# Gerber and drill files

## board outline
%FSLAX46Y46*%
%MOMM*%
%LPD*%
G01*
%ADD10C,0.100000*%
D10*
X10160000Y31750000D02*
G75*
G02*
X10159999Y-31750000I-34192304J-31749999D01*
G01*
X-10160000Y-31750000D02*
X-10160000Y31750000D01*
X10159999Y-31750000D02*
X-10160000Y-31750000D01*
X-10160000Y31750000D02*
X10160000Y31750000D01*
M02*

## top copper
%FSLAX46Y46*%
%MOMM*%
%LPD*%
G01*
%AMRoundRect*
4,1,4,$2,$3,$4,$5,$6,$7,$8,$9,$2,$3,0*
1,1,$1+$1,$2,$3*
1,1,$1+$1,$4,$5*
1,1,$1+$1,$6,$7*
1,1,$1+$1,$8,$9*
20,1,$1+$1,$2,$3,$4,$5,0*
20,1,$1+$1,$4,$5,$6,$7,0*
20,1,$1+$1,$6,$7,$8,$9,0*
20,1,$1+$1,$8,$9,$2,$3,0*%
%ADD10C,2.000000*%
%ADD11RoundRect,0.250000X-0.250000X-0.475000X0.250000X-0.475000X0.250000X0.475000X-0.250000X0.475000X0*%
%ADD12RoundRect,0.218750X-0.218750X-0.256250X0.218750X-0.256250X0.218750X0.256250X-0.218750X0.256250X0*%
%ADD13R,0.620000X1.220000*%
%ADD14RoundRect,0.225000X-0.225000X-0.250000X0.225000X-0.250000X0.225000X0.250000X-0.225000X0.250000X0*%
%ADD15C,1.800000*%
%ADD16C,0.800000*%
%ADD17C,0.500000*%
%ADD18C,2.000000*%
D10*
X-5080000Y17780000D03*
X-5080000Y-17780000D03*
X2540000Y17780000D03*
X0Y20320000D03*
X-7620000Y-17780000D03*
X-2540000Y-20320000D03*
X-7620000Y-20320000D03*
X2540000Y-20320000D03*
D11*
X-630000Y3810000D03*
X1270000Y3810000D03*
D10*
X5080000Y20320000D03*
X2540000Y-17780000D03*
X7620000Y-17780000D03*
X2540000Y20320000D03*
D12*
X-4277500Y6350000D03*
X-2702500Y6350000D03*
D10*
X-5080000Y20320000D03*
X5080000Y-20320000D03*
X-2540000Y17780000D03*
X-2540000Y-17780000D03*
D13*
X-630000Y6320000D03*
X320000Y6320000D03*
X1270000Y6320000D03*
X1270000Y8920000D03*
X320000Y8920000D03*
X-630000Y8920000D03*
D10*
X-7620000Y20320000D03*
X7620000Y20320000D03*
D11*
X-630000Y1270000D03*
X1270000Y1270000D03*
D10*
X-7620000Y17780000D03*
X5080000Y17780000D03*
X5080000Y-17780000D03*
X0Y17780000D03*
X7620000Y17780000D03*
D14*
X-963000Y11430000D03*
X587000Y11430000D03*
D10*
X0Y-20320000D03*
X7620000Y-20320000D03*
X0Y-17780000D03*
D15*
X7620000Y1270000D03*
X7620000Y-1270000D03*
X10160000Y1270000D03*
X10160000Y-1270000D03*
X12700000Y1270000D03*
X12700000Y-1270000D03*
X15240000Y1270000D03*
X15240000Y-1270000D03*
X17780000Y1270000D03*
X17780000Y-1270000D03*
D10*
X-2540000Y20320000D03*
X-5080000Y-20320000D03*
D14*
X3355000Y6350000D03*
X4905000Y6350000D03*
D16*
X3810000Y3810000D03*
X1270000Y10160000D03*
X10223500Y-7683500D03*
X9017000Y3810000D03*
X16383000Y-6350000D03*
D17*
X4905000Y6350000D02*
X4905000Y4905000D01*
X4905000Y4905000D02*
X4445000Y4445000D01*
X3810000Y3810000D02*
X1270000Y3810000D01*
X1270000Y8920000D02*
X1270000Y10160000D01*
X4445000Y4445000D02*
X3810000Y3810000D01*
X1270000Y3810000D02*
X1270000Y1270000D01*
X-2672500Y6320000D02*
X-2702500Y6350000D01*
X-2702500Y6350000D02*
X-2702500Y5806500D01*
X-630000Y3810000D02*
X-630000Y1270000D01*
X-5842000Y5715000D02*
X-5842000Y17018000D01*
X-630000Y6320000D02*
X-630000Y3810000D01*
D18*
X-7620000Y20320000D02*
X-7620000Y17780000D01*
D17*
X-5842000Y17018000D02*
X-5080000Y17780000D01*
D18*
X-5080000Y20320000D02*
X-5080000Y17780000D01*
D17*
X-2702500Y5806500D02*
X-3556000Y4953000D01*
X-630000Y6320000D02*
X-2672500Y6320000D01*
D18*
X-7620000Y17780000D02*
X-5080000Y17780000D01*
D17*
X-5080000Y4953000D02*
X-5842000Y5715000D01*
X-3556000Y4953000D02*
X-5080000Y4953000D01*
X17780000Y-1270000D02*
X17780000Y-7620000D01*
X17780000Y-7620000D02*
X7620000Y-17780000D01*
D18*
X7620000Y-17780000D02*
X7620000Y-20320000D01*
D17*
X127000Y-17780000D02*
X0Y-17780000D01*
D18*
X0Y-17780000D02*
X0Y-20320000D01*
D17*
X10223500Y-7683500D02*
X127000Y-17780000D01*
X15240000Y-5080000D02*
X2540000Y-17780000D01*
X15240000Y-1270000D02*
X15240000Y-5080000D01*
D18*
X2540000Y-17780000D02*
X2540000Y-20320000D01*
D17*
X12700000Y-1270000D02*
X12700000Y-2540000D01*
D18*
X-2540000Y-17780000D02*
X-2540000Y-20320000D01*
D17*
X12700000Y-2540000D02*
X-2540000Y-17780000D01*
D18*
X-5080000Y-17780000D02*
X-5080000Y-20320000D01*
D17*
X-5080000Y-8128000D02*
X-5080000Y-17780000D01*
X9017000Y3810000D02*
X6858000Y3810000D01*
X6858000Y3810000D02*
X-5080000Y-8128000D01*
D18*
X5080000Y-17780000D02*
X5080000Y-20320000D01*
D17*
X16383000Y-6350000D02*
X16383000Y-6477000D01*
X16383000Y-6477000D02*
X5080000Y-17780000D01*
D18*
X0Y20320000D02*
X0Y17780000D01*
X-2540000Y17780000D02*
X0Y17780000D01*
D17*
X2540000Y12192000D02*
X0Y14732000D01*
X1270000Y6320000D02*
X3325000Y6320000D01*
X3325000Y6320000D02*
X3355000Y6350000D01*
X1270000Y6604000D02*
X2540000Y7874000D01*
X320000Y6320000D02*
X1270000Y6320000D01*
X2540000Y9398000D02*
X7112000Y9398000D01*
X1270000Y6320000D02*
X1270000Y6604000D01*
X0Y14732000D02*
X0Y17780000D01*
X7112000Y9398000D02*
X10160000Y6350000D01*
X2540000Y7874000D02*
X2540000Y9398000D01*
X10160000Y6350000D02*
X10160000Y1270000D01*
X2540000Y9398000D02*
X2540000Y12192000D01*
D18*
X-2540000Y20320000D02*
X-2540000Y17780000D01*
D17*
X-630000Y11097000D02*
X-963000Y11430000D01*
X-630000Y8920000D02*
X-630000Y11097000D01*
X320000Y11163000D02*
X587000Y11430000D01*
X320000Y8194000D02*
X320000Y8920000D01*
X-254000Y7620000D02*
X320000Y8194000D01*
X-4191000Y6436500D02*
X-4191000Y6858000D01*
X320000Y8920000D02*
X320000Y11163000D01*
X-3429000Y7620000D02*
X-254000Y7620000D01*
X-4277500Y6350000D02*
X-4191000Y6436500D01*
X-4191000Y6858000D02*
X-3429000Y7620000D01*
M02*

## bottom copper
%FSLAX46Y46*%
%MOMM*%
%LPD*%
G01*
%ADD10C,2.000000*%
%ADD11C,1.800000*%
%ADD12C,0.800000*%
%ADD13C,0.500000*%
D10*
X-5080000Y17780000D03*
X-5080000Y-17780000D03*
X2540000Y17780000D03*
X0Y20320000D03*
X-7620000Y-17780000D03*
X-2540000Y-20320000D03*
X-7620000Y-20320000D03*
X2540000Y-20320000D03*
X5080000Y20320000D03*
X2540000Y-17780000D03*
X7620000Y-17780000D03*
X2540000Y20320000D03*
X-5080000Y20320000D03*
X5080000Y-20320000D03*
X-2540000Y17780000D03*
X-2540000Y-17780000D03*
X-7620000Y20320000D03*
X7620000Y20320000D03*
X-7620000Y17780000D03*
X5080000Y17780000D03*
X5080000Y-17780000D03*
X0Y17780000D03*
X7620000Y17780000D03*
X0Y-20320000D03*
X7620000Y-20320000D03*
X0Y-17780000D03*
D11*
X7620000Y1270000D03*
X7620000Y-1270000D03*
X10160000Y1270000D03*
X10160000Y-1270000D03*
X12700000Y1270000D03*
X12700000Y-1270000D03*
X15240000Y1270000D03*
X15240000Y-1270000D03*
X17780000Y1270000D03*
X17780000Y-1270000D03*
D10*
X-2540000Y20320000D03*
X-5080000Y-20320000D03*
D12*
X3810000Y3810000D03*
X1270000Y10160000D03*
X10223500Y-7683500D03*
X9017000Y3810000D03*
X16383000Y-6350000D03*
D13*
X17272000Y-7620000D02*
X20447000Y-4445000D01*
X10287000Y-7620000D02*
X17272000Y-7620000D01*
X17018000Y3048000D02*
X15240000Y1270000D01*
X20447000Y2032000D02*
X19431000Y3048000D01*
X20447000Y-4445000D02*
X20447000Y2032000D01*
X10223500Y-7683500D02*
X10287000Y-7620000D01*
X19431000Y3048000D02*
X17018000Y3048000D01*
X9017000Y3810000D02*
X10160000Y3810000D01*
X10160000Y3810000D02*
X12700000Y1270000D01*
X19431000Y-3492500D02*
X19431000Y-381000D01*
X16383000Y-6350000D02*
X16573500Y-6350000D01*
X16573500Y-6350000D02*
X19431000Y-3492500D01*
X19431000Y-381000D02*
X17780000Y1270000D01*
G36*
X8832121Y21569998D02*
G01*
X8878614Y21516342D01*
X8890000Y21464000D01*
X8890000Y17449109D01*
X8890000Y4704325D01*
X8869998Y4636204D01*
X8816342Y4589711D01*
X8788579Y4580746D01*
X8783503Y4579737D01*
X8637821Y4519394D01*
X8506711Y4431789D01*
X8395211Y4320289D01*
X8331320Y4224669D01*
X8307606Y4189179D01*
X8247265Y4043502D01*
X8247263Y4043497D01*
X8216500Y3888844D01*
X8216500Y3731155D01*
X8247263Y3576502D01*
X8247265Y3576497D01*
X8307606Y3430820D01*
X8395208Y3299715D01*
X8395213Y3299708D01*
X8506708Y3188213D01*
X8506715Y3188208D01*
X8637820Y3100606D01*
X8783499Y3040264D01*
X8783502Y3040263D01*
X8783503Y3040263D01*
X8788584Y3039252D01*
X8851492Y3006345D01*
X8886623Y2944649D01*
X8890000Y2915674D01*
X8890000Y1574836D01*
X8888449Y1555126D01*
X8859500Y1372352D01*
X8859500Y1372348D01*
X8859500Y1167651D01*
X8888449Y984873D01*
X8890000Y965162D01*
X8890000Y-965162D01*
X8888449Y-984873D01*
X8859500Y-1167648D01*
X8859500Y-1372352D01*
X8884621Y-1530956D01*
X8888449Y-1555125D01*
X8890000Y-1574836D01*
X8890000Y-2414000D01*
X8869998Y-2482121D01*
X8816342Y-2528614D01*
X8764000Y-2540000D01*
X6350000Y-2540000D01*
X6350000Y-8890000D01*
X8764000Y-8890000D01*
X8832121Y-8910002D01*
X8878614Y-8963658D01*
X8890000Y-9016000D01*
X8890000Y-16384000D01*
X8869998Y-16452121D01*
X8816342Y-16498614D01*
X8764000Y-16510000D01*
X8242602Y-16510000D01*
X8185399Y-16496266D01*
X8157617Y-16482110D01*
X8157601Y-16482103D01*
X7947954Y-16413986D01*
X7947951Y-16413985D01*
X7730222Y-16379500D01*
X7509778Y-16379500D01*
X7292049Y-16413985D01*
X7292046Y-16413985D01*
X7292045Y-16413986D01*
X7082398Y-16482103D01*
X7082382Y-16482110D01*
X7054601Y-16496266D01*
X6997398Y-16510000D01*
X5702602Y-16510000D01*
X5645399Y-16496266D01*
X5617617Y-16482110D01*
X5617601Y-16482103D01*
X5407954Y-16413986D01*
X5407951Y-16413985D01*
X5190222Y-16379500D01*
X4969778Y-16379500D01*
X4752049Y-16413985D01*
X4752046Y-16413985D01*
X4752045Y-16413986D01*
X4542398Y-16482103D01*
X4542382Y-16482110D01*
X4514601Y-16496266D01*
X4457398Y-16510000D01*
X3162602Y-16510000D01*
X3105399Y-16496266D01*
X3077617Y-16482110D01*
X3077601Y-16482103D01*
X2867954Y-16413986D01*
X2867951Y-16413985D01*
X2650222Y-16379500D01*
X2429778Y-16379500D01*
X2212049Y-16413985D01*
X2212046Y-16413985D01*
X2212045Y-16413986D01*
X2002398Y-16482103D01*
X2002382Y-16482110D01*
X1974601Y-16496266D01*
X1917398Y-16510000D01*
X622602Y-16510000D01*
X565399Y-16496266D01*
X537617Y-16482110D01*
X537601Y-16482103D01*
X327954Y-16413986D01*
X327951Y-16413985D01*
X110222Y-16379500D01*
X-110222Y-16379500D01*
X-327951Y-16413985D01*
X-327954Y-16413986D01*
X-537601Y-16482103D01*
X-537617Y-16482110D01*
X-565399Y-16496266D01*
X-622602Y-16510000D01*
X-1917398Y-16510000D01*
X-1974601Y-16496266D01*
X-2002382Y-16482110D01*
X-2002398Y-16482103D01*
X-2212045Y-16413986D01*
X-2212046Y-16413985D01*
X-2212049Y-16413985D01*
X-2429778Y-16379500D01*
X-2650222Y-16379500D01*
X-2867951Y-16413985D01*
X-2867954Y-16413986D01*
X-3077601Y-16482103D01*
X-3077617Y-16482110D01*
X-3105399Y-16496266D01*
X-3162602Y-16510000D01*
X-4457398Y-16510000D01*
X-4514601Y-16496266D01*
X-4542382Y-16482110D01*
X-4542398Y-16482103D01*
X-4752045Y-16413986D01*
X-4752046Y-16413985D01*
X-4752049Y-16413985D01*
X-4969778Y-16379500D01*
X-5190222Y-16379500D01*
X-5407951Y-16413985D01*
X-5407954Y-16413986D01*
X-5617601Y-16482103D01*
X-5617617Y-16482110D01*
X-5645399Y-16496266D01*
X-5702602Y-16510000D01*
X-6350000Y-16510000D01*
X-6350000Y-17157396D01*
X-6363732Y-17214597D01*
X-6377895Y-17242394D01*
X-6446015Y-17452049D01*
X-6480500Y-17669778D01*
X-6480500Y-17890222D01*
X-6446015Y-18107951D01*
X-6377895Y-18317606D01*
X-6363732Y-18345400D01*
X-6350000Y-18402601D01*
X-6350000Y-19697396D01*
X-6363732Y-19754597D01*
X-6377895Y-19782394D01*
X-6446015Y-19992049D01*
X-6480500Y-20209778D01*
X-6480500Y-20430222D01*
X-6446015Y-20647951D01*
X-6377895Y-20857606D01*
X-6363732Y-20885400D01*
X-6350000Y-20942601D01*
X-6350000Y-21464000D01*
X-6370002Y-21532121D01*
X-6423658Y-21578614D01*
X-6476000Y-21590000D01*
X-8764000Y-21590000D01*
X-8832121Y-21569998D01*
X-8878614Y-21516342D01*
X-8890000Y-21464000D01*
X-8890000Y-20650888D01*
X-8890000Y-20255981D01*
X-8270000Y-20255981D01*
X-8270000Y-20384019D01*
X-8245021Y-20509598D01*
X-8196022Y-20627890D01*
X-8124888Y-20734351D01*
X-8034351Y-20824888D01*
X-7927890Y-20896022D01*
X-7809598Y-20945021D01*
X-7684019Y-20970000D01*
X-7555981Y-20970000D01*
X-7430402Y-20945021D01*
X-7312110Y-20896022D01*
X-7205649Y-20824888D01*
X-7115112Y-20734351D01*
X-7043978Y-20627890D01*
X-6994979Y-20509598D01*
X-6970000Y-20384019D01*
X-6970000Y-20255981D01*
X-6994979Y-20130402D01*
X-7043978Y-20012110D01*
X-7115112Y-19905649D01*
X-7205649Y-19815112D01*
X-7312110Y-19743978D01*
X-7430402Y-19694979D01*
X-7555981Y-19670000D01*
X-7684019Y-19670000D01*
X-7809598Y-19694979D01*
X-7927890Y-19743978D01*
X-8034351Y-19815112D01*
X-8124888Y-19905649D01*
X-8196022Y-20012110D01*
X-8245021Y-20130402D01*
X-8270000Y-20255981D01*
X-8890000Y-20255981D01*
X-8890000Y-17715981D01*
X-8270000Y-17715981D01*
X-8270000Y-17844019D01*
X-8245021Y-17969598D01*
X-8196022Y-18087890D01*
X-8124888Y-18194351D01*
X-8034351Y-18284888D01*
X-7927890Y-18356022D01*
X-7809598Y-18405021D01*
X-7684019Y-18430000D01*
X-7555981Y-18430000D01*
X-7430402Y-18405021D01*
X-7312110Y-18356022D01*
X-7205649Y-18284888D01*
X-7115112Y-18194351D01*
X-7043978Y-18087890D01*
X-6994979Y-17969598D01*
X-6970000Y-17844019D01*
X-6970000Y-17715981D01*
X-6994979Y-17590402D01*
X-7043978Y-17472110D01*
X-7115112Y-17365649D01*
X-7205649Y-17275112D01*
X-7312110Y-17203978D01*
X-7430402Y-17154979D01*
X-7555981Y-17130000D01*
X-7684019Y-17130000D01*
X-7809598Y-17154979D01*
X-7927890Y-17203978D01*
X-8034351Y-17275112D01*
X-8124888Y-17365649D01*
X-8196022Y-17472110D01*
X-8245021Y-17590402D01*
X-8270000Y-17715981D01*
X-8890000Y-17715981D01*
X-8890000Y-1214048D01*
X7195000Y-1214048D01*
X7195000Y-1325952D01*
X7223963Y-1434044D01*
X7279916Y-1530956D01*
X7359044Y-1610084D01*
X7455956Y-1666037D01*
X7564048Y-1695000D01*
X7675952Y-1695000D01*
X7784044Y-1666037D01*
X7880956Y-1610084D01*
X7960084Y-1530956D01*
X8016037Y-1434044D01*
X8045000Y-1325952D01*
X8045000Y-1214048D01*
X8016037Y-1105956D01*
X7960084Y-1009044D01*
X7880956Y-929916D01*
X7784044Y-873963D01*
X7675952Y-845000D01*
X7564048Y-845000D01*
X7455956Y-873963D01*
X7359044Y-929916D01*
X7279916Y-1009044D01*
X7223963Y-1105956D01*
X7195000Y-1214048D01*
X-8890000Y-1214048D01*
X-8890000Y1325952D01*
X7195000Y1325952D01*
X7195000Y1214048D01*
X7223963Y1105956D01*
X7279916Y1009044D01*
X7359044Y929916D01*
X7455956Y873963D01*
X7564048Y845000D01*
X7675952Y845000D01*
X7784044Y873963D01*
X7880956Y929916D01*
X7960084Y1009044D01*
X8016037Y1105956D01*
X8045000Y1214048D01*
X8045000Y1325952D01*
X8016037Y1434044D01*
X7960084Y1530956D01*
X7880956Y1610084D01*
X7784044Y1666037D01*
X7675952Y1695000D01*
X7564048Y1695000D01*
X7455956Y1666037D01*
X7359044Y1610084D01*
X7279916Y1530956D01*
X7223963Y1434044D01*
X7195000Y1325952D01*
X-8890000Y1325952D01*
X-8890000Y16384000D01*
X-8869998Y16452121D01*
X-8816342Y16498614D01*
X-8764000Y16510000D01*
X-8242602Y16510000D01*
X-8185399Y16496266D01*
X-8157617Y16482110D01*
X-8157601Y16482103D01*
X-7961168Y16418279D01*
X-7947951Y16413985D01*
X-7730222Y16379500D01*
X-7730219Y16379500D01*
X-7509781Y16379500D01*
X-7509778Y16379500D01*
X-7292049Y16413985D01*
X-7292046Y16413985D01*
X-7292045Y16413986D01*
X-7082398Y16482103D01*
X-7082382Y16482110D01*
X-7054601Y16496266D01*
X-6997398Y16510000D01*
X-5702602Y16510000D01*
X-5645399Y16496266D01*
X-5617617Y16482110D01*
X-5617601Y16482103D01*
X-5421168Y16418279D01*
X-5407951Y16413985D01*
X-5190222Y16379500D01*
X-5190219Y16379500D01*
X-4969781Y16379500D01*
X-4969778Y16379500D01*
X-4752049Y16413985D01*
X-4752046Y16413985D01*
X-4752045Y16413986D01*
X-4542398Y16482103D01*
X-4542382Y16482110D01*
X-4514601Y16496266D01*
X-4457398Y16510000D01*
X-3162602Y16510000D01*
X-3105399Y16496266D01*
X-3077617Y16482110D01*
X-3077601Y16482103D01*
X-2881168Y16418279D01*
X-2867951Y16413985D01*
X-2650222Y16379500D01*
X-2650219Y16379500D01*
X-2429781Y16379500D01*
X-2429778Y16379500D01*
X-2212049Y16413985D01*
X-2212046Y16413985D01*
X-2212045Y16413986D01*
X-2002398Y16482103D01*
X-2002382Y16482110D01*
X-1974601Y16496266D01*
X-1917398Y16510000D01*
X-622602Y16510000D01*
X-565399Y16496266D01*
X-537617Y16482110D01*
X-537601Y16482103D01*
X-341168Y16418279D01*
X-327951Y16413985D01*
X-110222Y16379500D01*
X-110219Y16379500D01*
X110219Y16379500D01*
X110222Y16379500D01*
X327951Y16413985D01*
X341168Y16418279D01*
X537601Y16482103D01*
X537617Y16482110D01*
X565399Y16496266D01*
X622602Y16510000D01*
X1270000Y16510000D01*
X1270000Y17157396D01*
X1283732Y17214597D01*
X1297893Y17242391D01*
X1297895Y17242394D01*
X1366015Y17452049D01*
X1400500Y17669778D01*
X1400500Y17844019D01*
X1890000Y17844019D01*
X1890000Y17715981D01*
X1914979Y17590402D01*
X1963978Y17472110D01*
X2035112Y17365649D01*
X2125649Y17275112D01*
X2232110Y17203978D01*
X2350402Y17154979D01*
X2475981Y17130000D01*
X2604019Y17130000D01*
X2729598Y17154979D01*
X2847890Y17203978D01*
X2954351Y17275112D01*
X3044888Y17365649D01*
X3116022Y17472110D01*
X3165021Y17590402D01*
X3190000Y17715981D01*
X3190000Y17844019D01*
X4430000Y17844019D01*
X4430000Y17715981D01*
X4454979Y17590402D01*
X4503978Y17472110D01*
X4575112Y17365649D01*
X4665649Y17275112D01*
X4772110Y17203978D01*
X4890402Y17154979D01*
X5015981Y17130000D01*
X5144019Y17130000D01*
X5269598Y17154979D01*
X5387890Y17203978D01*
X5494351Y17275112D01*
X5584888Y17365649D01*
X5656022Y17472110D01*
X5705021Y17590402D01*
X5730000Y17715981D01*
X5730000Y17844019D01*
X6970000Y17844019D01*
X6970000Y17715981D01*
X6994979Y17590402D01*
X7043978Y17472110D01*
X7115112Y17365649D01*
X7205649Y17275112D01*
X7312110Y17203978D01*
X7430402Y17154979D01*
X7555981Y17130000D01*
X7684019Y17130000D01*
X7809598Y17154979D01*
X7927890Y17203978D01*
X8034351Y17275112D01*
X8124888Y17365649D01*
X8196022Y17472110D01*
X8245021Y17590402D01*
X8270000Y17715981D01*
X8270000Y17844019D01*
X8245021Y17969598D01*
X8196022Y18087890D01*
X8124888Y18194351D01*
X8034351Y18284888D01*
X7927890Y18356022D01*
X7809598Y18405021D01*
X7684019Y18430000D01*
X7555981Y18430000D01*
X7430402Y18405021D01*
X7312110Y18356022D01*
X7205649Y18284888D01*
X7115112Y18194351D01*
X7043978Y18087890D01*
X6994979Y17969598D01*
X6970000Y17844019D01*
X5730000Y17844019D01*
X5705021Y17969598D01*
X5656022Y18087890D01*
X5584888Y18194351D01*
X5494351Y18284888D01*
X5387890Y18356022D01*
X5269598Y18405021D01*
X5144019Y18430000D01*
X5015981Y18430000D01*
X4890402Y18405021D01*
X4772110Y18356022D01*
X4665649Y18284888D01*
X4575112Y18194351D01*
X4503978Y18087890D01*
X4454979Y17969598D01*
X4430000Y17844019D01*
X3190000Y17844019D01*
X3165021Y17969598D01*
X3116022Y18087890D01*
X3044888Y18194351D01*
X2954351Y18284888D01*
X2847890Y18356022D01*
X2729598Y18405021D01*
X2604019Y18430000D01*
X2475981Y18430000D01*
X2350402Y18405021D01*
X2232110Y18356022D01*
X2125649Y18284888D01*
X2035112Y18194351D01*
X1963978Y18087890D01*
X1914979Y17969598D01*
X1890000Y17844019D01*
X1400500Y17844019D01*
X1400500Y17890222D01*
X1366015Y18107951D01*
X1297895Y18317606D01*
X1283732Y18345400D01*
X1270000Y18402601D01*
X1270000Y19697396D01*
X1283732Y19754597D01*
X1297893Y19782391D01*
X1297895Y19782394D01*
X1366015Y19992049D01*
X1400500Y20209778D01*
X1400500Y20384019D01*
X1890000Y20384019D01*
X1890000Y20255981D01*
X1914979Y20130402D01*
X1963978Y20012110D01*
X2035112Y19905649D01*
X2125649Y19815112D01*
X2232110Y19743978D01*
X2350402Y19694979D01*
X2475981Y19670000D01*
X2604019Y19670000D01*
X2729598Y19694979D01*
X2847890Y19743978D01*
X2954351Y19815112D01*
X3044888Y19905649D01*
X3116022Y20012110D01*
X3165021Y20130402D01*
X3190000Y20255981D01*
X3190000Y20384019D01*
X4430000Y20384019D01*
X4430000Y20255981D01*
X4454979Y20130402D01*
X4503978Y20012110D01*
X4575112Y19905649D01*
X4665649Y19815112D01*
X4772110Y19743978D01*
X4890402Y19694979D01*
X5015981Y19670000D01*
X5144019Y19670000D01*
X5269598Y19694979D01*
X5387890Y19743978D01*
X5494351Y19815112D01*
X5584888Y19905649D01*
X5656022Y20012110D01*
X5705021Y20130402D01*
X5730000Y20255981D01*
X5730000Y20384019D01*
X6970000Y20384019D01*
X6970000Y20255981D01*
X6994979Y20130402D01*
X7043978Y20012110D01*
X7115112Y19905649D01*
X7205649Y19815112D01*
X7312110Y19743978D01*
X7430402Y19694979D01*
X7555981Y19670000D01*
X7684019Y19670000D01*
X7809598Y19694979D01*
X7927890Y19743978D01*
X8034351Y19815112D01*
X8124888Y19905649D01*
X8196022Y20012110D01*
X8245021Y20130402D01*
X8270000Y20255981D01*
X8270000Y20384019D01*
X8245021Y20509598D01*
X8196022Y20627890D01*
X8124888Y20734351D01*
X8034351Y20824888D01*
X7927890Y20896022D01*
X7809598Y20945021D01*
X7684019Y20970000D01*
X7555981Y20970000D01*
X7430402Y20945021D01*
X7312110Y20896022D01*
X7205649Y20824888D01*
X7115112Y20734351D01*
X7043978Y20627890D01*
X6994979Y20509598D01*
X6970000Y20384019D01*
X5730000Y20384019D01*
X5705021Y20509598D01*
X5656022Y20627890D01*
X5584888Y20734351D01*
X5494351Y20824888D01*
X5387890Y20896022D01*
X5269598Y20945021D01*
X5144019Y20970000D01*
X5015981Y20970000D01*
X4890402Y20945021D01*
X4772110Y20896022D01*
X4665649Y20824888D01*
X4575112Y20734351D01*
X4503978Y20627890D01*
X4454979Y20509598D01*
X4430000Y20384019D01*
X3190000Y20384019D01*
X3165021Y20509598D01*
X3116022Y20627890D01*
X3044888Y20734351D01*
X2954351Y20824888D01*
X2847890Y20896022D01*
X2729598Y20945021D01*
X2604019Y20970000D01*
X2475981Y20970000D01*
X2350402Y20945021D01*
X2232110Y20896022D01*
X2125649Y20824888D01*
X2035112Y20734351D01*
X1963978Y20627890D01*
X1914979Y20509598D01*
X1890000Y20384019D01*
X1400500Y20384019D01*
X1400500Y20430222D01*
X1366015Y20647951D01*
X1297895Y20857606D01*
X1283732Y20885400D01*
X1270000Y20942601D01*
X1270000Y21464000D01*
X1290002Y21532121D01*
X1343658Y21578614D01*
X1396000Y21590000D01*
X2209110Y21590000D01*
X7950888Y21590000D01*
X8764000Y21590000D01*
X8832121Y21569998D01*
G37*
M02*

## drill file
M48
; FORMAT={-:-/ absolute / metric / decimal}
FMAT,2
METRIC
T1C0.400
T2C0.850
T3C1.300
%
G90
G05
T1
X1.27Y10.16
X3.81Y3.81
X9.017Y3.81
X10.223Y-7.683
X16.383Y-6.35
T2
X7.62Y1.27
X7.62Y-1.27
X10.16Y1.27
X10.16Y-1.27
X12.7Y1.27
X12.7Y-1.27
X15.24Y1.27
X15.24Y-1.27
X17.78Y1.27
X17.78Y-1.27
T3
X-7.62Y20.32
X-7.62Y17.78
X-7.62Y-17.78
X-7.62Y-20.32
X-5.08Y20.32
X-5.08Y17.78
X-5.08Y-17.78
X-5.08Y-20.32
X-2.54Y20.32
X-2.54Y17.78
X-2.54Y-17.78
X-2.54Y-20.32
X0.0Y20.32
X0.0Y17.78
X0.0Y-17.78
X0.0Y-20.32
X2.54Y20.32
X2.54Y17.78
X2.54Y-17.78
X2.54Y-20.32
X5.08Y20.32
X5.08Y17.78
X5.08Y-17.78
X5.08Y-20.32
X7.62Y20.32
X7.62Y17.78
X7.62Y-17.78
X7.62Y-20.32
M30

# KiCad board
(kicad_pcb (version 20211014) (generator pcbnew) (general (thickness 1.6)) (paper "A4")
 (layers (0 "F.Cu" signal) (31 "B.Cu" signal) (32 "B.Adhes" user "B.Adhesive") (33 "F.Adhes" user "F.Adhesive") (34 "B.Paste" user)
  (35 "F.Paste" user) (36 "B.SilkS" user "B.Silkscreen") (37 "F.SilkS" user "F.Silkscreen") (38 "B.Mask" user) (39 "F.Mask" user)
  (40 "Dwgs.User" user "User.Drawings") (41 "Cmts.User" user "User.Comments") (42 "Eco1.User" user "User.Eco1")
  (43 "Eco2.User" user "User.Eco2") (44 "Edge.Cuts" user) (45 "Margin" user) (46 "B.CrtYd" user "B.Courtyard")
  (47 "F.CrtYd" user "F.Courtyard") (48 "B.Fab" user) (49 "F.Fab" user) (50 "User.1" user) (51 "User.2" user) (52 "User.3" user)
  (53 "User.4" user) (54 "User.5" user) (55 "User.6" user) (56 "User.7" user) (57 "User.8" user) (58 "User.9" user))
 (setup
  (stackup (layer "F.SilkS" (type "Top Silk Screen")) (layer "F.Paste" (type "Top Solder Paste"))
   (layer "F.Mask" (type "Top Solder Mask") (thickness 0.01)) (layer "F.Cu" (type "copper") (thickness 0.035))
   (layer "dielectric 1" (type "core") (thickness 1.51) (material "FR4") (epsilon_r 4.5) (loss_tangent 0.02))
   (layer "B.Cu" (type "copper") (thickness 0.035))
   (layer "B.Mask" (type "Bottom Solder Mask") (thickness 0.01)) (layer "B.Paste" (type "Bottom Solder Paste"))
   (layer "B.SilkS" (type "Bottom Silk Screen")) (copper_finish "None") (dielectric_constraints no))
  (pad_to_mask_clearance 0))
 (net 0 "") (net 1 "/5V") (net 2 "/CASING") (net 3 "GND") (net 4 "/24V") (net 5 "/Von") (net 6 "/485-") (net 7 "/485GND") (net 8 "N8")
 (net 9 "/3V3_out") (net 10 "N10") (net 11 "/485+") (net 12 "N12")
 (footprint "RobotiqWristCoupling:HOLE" (layer "F.Cu") (at -5.08 -17.78)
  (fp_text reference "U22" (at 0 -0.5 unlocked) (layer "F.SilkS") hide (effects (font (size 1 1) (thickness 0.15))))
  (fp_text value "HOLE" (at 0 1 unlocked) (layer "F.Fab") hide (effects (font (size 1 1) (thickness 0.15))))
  (pad "1" thru_hole circle (at 0 0) (size 2 2) (drill 1.3) (layers *.Cu *.Mask) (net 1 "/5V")))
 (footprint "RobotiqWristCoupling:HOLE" (layer "F.Cu") (at -5.08 17.78)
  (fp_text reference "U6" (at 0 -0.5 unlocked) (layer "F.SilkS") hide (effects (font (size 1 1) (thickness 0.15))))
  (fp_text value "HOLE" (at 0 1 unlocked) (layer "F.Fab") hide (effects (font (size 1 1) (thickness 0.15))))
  (pad "1" thru_hole circle (at 0 0) (size 2 2) (drill 1.3) (layers *.Cu *.Mask) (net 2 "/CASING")))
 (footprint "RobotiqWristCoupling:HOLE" (layer "F.Cu") (at 2.54 -17.78)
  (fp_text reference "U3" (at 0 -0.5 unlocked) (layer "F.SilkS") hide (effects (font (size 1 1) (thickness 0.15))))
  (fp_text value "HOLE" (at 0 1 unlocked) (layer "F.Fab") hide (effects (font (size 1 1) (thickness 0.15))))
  (pad "1" thru_hole circle (at 0 0) (size 2 2) (drill 1.3) (layers *.Cu *.Mask) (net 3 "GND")))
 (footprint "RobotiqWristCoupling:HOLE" (layer "F.Cu") (at 0 -20.32)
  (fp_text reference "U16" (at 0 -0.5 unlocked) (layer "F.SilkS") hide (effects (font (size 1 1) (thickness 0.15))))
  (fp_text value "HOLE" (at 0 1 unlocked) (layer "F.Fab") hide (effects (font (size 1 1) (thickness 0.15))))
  (pad "1" thru_hole circle (at 0 0) (size 2 2) (drill 1.3) (layers *.Cu *.Mask) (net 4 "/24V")))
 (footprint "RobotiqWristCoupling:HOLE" (layer "F.Cu") (at -7.62 17.78)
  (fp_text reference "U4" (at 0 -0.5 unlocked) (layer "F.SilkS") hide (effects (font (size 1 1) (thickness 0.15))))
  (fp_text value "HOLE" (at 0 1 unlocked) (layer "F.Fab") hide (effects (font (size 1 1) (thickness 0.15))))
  (pad "1" thru_hole circle (at 0 0) (size 2 2) (drill 1.3) (layers *.Cu *.Mask) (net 3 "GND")))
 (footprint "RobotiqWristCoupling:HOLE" (layer "F.Cu") (at -2.54 20.32)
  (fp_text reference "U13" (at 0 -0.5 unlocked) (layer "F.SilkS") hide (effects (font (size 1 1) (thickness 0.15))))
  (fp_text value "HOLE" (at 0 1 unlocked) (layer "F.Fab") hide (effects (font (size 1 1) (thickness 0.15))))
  (pad "1" thru_hole circle (at 0 0) (size 2 2) (drill 1.3) (layers *.Cu *.Mask) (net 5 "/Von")))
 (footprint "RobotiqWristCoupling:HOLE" (layer "F.Cu") (at -7.62 20.32)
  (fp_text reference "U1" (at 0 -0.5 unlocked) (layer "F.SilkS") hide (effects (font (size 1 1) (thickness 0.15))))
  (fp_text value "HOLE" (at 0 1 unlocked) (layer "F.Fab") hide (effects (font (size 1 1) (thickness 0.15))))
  (pad "1" thru_hole circle (at 0 0) (size 2 2) (drill 1.3) (layers *.Cu *.Mask) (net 3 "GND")))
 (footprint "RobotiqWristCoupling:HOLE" (layer "F.Cu") (at 2.54 20.32)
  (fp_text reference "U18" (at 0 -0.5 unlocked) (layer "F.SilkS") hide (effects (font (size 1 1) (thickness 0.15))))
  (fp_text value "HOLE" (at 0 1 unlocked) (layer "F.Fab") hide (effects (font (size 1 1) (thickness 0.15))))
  (pad "1" thru_hole circle (at 0 0) (size 2 2) (drill 1.3) (layers *.Cu *.Mask) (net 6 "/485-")))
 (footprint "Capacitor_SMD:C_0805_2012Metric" (layer "F.Cu") (at 0.32 -3.81)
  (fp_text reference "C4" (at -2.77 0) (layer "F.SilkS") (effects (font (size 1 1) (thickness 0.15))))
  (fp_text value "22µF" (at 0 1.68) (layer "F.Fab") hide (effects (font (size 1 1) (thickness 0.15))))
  (pad "1" smd roundrect (at -0.95 0) (size 1 1.45) (layers "F.Cu" "F.Paste" "F.Mask") (roundrect_rratio 0.25) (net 1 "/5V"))
  (pad "2" smd roundrect (at 0.95 0) (size 1 1.45) (layers "F.Cu" "F.Paste" "F.Mask") (roundrect_rratio 0.25) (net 3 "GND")))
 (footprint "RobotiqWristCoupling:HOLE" (layer "F.Cu") (at 5.08 -20.32)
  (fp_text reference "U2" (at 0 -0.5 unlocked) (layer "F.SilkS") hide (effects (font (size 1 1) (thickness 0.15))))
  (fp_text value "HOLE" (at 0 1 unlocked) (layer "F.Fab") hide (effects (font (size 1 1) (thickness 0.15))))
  (pad "1" thru_hole circle (at 0 0) (size 2 2) (drill 1.3) (layers *.Cu *.Mask) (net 3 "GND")))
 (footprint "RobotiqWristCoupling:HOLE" (layer "F.Cu") (at 2.54 17.78)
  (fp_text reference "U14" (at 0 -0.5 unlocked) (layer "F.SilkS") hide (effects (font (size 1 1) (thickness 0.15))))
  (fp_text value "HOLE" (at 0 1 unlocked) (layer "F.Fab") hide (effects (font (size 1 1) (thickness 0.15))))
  (pad "1" thru_hole circle (at 0 0) (size 2 2) (drill 1.3) (layers *.Cu *.Mask) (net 6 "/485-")))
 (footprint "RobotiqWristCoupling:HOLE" (layer "F.Cu") (at 7.62 17.78)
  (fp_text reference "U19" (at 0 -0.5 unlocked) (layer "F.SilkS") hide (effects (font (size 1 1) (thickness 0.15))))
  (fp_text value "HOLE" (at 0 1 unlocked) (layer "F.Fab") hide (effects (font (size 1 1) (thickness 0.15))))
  (pad "1" thru_hole circle (at 0 0) (size 2 2) (drill 1.3) (layers *.Cu *.Mask) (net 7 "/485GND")))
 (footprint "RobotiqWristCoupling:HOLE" (layer "F.Cu") (at 2.54 -20.32)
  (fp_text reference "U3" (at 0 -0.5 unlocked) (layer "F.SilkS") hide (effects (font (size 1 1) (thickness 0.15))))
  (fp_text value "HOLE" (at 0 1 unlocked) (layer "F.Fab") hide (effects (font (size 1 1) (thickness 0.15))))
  (pad "1" thru_hole circle (at 0 0) (size 2 2) (drill 1.3) (layers *.Cu *.Mask) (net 3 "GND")))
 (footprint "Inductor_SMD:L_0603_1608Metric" (layer "F.Cu") (at -3.49 -6.35)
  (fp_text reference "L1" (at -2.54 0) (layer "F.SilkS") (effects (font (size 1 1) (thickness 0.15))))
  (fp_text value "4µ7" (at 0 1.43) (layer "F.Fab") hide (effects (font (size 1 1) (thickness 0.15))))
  (pad "1" smd roundrect (at -0.7875 0) (size 0.875 0.95) (layers "F.Cu" "F.Paste" "F.Mask") (roundrect_rratio 0.25) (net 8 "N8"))
  (pad "2" smd roundrect (at 0.7875 0) (size 0.875 0.95) (layers "F.Cu" "F.Paste" "F.Mask") (roundrect_rratio 0.25) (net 1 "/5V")))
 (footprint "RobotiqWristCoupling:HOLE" (layer "F.Cu") (at -5.08 -20.32)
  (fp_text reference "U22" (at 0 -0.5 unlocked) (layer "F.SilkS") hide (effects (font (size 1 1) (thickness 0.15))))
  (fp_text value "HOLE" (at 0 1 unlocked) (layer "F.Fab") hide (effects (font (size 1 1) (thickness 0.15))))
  (pad "1" thru_hole circle (at 0 0) (size 2 2) (drill 1.3) (layers *.Cu *.Mask) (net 1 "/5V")))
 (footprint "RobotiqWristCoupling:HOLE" (layer "F.Cu") (at 5.08 20.32)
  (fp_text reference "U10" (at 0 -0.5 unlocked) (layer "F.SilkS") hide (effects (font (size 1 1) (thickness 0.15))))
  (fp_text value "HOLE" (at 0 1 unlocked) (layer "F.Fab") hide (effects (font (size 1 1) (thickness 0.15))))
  (pad "1" thru_hole circle (at 0 0) (size 2 2) (drill 1.3) (layers *.Cu *.Mask) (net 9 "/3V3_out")))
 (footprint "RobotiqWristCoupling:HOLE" (layer "F.Cu") (at -2.54 -17.78)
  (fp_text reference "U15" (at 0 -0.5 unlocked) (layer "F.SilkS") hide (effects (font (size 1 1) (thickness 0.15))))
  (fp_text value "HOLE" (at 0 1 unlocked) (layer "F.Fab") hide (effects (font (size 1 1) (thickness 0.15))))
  (pad "1" thru_hole circle (at 0 0) (size 2 2) (drill 1.3) (layers *.Cu *.Mask) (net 4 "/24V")))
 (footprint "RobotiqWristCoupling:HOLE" (layer "F.Cu") (at -2.54 17.78)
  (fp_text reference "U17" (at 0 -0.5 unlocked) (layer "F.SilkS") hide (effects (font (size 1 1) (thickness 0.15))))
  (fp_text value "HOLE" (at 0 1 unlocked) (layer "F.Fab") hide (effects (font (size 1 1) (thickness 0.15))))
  (pad "1" thru_hole circle (at 0 0) (size 2 2) (drill 1.3) (layers *.Cu *.Mask) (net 5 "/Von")))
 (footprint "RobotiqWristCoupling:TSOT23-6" (layer "F.Cu") (at 0.32 -7.62)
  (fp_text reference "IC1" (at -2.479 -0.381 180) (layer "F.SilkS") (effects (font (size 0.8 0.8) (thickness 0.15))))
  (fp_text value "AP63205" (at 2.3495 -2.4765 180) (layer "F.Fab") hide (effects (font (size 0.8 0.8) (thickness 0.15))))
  (pad "1" smd rect (at -0.95 1.3) (size 0.62 1.22) (layers "F.Cu" "F.Paste" "F.Mask") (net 1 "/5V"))
  (pad "2" smd rect (at 0 1.3) (size 0.62 1.22) (layers "F.Cu" "F.Paste" "F.Mask") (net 4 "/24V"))
  (pad "3" smd rect (at 0.95 1.3) (size 0.62 1.22) (layers "F.Cu" "F.Paste" "F.Mask") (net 4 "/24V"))
  (pad "4" smd rect (at 0.95 -1.3) (size 0.62 1.22) (layers "F.Cu" "F.Paste" "F.Mask") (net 3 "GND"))
  (pad "5" smd rect (at 0 -1.3) (size 0.62 1.22) (layers "F.Cu" "F.Paste" "F.Mask") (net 8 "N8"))
  (pad "6" smd rect (at -0.95 -1.3) (size 0.62 1.22) (layers "F.Cu" "F.Paste" "F.Mask") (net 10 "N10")))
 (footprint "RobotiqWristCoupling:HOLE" (layer "F.Cu") (at -7.62 -20.32)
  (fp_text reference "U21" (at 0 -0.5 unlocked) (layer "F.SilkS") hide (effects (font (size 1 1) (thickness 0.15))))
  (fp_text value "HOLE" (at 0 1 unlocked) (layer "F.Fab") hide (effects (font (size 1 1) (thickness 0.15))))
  (pad "1" thru_hole circle (at 0 0) (size 2 2) (drill 1.3) (layers *.Cu *.Mask) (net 1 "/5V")))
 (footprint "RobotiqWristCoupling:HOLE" (layer "F.Cu") (at 7.62 -20.32)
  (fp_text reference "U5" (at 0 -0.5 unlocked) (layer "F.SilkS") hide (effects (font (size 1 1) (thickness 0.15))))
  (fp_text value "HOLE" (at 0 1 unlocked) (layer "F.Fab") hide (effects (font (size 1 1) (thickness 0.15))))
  (pad "1" thru_hole circle (at 0 0) (size 2 2) (drill 1.3) (layers *.Cu *.Mask) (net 3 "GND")))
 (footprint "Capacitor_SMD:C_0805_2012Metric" (layer "F.Cu") (at 0.32 -1.27)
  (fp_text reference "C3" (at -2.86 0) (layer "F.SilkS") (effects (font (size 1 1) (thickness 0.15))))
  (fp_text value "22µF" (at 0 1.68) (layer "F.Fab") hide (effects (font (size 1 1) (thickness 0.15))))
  (pad "1" smd roundrect (at -0.95 0) (size 1 1.45) (layers "F.Cu" "F.Paste" "F.Mask") (roundrect_rratio 0.25) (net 1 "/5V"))
  (pad "2" smd roundrect (at 0.95 0) (size 1 1.45) (layers "F.Cu" "F.Paste" "F.Mask") (roundrect_rratio 0.25) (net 3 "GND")))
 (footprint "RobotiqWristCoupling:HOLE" (layer "F.Cu") (at -7.62 -17.78)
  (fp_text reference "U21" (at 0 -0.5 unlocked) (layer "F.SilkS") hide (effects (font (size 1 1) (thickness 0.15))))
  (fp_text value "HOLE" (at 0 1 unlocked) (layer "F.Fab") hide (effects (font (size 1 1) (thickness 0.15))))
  (pad "1" thru_hole circle (at 0 0) (size 2 2) (drill 1.3) (layers *.Cu *.Mask) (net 1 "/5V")))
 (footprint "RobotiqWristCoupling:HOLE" (layer "F.Cu") (at 5.08 -17.78)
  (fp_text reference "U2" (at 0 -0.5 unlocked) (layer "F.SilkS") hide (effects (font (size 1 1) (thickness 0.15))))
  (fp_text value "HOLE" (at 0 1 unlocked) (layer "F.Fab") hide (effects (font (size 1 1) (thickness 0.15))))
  (pad "1" thru_hole circle (at 0 0) (size 2 2) (drill 1.3) (layers *.Cu *.Mask) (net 3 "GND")))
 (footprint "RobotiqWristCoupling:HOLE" (layer "F.Cu") (at 5.08 17.78)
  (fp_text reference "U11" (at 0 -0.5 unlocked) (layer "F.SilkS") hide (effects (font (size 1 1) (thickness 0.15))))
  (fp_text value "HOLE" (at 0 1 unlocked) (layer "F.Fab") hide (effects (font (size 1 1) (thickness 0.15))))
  (pad "1" thru_hole circle (at 0 0) (size 2 2) (drill 1.3) (layers *.Cu *.Mask) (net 9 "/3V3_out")))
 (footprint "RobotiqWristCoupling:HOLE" (layer "F.Cu") (at 0 -17.78)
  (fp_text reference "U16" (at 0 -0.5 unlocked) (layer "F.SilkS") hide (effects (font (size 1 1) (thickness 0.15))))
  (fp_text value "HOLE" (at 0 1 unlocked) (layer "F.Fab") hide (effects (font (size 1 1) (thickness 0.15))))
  (pad "1" thru_hole circle (at 0 0) (size 2 2) (drill 1.3) (layers *.Cu *.Mask) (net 4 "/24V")))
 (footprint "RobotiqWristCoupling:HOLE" (layer "F.Cu") (at 7.62 -17.78)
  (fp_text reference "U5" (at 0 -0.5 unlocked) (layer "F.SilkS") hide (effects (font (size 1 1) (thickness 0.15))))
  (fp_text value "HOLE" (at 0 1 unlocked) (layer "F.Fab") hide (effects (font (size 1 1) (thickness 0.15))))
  (pad "1" thru_hole circle (at 0 0) (size 2 2) (drill 1.3) (layers *.Cu *.Mask) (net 3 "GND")))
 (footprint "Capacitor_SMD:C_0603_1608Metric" (layer "F.Cu") (at -0.188 -11.43)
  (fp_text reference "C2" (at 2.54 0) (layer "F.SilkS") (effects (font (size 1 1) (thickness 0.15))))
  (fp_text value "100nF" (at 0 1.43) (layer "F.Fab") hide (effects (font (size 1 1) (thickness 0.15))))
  (pad "1" smd roundrect (at -0.775 0) (size 0.9 0.95) (layers "F.Cu" "F.Paste" "F.Mask") (roundrect_rratio 0.25) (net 10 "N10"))
  (pad "2" smd roundrect (at 0.775 0) (size 0.9 0.95) (layers "F.Cu" "F.Paste" "F.Mask") (roundrect_rratio 0.25) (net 8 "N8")))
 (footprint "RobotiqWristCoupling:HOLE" (layer "F.Cu") (at 0 20.32)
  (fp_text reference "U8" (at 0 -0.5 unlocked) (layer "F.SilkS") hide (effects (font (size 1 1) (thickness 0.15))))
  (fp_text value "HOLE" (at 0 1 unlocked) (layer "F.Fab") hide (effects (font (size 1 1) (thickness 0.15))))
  (pad "1" thru_hole circle (at 0 0) (size 2 2) (drill 1.3) (layers *.Cu *.Mask) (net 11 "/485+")))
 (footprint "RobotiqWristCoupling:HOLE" (layer "F.Cu") (at 7.62 20.32)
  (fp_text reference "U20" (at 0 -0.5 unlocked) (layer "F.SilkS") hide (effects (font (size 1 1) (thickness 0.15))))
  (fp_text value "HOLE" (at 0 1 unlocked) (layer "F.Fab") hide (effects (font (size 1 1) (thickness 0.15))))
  (pad "1" thru_hole circle (at 0 0) (size 2 2) (drill 1.3) (layers *.Cu *.Mask) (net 7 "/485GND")))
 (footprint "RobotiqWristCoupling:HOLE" (layer "F.Cu") (at 0 17.78)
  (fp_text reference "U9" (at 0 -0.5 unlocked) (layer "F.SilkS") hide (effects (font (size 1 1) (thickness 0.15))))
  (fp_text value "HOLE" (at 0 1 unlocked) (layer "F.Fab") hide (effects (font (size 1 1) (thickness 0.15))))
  (pad "1" thru_hole circle (at 0 0) (size 2 2) (drill 1.3) (layers *.Cu *.Mask) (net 11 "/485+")))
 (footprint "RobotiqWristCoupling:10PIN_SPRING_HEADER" (layer "F.Cu") (at 7.62 1.27)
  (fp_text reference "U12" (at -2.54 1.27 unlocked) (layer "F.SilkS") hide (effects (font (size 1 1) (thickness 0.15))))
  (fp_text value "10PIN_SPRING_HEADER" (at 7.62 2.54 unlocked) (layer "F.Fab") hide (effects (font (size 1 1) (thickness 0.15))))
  (pad "1" thru_hole circle (at 0 -2.54) (size 1.8 1.8) (drill 0.85) (layers *.Cu *.Mask) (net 3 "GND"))
  (pad "2" thru_hole circle (at 0 0) (size 1.8 1.8) (drill 0.85) (layers *.Cu *.Mask) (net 3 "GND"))
  (pad "3" thru_hole circle (at 2.54 -2.54) (size 1.8 1.8) (drill 0.85) (layers *.Cu *.Mask) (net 4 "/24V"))
  (pad "4" thru_hole circle (at 2.54 0) (size 1.8 1.8) (drill 0.85) (layers *.Cu *.Mask) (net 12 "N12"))
  (pad "5" thru_hole circle (at 5.08 -2.54) (size 1.8 1.8) (drill 0.85) (layers *.Cu *.Mask) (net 2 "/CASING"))
  (pad "6" thru_hole circle (at 5.08 0) (size 1.8 1.8) (drill 0.85) (layers *.Cu *.Mask) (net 5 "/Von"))
  (pad "7" thru_hole circle (at 7.62 -2.54) (size 1.8 1.8) (drill 0.85) (layers *.Cu *.Mask) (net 11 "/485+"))
  (pad "8" thru_hole circle (at 7.62 0) (size 1.8 1.8) (drill 0.85) (layers *.Cu *.Mask) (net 6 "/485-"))
  (pad "9" thru_hole circle (at 10.16 -2.54) (size 1.8 1.8) (drill 0.85) (layers *.Cu *.Mask) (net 9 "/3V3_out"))
  (pad "10" thru_hole circle (at 10.16 0) (size 1.8 1.8) (drill 0.85) (layers *.Cu *.Mask) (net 7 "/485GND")))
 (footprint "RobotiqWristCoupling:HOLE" (layer "F.Cu") (at -2.54 -20.32)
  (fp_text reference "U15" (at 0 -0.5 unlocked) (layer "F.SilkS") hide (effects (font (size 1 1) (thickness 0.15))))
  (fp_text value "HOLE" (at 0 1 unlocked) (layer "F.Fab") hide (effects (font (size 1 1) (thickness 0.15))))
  (pad "1" thru_hole circle (at 0 0) (size 2 2) (drill 1.3) (layers *.Cu *.Mask) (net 4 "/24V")))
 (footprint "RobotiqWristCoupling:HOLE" (layer "F.Cu") (at -5.08 20.32)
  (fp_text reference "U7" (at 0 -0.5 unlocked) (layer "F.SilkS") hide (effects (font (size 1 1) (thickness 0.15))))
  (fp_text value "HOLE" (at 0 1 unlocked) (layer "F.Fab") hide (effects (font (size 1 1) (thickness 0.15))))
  (pad "1" thru_hole circle (at 0 0) (size 2 2) (drill 1.3) (layers *.Cu *.Mask) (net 2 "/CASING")))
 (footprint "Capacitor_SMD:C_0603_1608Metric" (layer "F.Cu") (at 4.13 -6.35)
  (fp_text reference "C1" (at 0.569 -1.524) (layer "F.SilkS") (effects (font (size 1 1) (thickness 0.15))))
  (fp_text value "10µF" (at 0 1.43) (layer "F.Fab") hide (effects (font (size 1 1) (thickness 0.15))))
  (pad "1" smd roundrect (at -0.775 0) (size 0.9 0.95) (layers "F.Cu" "F.Paste" "F.Mask") (roundrect_rratio 0.25) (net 4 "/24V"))
  (pad "2" smd roundrect (at 0.775 0) (size 0.9 0.95) (layers "F.Cu" "F.Paste" "F.Mask") (roundrect_rratio 0.25) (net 3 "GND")))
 (gr_arc (start 10.16 -31.75) (mid 22.627916 0) (end 10.159999 31.75) (layer "Edge.Cuts") (width 0.1))
 (gr_line (start -10.16 31.75) (end -10.16 -31.75) (layer "Edge.Cuts") (width 0.1))
 (gr_line (start 10.159999 31.75) (end -10.16 31.75) (layer "Edge.Cuts") (width 0.1))
 (gr_line (start -10.16 -31.75) (end 10.16 -31.75) (layer "Edge.Cuts") (width 0.1))
 (segment (start 4.905 -6.35) (end 4.905 -4.905) (width 0.5) (layer "F.Cu") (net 3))
 (segment (start 4.905 -4.905) (end 4.445 -4.445) (width 0.5) (layer "F.Cu") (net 3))
 (segment (start 3.81 -3.81) (end 1.27 -3.81) (width 0.5) (layer "F.Cu") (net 3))
 (segment (start 1.27 -8.92) (end 1.27 -10.16) (width 0.5) (layer "F.Cu") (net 3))
 (segment (start 4.445 -4.445) (end 3.81 -3.81) (width 0.5) (layer "F.Cu") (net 3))
 (segment (start 1.27 -3.81) (end 1.27 -1.27) (width 0.5) (layer "F.Cu") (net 3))
 (via (at 3.81 -3.81) (size 0.8) (drill 0.4) (layers "F.Cu" "B.Cu") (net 3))
 (via (at 1.27 -10.16) (size 0.8) (drill 0.4) (layers "F.Cu" "B.Cu") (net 3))
 (segment (start -2.6725 -6.32) (end -2.7025 -6.35) (width 0.5) (layer "F.Cu") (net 1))
 (segment (start -2.7025 -6.35) (end -2.7025 -5.8065) (width 0.5) (layer "F.Cu") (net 1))
 (segment (start -0.63 -3.81) (end -0.63 -1.27) (width 0.5) (layer "F.Cu") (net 1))
 (segment (start -5.842 -5.715) (end -5.842 -17.018) (width 0.5) (layer "F.Cu") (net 1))
 (segment (start -0.63 -6.32) (end -0.63 -3.81) (width 0.5) (layer "F.Cu") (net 1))
 (segment (start -7.62 -20.32) (end -7.62 -17.78) (width 2) (layer "F.Cu") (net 1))
 (segment (start -5.842 -17.018) (end -5.08 -17.78) (width 0.5) (layer "F.Cu") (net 1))
 (segment (start -5.08 -20.32) (end -5.08 -17.78) (width 2) (layer "F.Cu") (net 1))
 (segment (start -2.7025 -5.8065) (end -3.556 -4.953) (width 0.5) (layer "F.Cu") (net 1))
 (segment (start -0.63 -6.32) (end -2.6725 -6.32) (width 0.5) (layer "F.Cu") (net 1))
 (segment (start -7.62 -17.78) (end -5.08 -17.78) (width 2) (layer "F.Cu") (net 1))
 (segment (start -5.08 -4.953) (end -5.842 -5.715) (width 0.5) (layer "F.Cu") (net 1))
 (segment (start -3.556 -4.953) (end -5.08 -4.953) (width 0.5) (layer "F.Cu") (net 1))
 (segment (start 17.78 1.27) (end 17.78 7.62) (width 0.5) (layer "F.Cu") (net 7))
 (segment (start 17.78 7.62) (end 7.62 17.78) (width 0.5) (layer "F.Cu") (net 7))
 (segment (start 7.62 17.78) (end 7.62 20.32) (width 2) (layer "F.Cu") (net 7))
 (segment (start 0.127 17.78) (end 0 17.78) (width 0.5) (layer "F.Cu") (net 11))
 (segment (start 0 17.78) (end 0 20.32) (width 2) (layer "F.Cu") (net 11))
 (segment (start 10.2235 7.6835) (end 0.127 17.78) (width 0.5) (layer "F.Cu") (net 11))
 (via (at 10.2235 7.6835) (size 0.8) (drill 0.4) (layers "F.Cu" "B.Cu") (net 11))
 (segment (start 17.272 7.62) (end 20.447 4.445) (width 0.5) (layer "B.Cu") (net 11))
 (segment (start 10.287 7.62) (end 17.272 7.62) (width 0.5) (layer "B.Cu") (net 11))
 (segment (start 17.018 -3.048) (end 15.24 -1.27) (width 0.5) (layer "B.Cu") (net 11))
 (segment (start 20.447 -2.032) (end 19.431 -3.048) (width 0.5) (layer "B.Cu") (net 11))
 (segment (start 20.447 4.445) (end 20.447 -2.032) (width 0.5) (layer "B.Cu") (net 11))
 (segment (start 10.2235 7.6835) (end 10.287 7.62) (width 0.5) (layer "B.Cu") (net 11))
 (segment (start 19.431 -3.048) (end 17.018 -3.048) (width 0.5) (layer "B.Cu") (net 11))
 (segment (start 15.24 5.08) (end 2.54 17.78) (width 0.5) (layer "F.Cu") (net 6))
 (segment (start 15.24 1.27) (end 15.24 5.08) (width 0.5) (layer "F.Cu") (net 6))
 (segment (start 2.54 17.78) (end 2.54 20.32) (width 2) (layer "F.Cu") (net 6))
 (segment (start 12.7 1.27) (end 12.7 2.54) (width 0.5) (layer "F.Cu") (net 5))
 (segment (start -2.54 17.78) (end -2.54 20.32) (width 2) (layer "F.Cu") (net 5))
 (segment (start 12.7 2.54) (end -2.54 17.78) (width 0.5) (layer "F.Cu") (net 5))
 (segment (start -5.08 17.78) (end -5.08 20.32) (width 2) (layer "F.Cu") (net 2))
 (segment (start -5.08 8.128) (end -5.08 17.78) (width 0.5) (layer "F.Cu") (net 2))
 (segment (start 9.017 -3.81) (end 6.858 -3.81) (width 0.5) (layer "F.Cu") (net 2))
 (segment (start 6.858 -3.81) (end -5.08 8.128) (width 0.5) (layer "F.Cu") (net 2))
 (via (at 9.017 -3.81) (size 0.8) (drill 0.4) (layers "F.Cu" "B.Cu") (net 2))
 (segment (start 9.017 -3.81) (end 10.16 -3.81) (width 0.5) (layer "B.Cu") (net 2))
 (segment (start 10.16 -3.81) (end 12.7 -1.27) (width 0.5) (layer "B.Cu") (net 2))
 (segment (start 5.08 17.78) (end 5.08 20.32) (width 2) (layer "F.Cu") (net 9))
 (segment (start 16.383 6.35) (end 16.383 6.477) (width 0.5) (layer "F.Cu") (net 9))
 (segment (start 16.383 6.477) (end 5.08 17.78) (width 0.5) (layer "F.Cu") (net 9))
 (via (at 16.383 6.35) (size 0.8) (drill 0.4) (layers "F.Cu" "B.Cu") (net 9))
 (segment (start 19.431 3.4925) (end 19.431 0.381) (width 0.5) (layer "B.Cu") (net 9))
 (segment (start 16.383 6.35) (end 16.5735 6.35) (width 0.5) (layer "B.Cu") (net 9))
 (segment (start 16.5735 6.35) (end 19.431 3.4925) (width 0.5) (layer "B.Cu") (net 9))
 (segment (start 19.431 0.381) (end 17.78 -1.27) (width 0.5) (layer "B.Cu") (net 9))
 (segment (start 0 -20.32) (end 0 -17.78) (width 2) (layer "F.Cu") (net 4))
 (segment (start -2.54 -17.78) (end 0 -17.78) (width 2) (layer "F.Cu") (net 4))
 (segment (start 2.54 -12.192) (end 0 -14.732) (width 0.5) (layer "F.Cu") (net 4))
 (segment (start 1.27 -6.32) (end 3.325 -6.32) (width 0.5) (layer "F.Cu") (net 4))
 (segment (start 3.325 -6.32) (end 3.355 -6.35) (width 0.5) (layer "F.Cu") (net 4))
 (segment (start 1.27 -6.604) (end 2.54 -7.874) (width 0.5) (layer "F.Cu") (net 4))
 (segment (start 0.32 -6.32) (end 1.27 -6.32) (width 0.5) (layer "F.Cu") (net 4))
 (segment (start 2.54 -9.398) (end 7.112 -9.398) (width 0.5) (layer "F.Cu") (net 4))
 (segment (start 1.27 -6.32) (end 1.27 -6.604) (width 0.5) (layer "F.Cu") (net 4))
 (segment (start 0 -14.732) (end 0 -17.78) (width 0.5) (layer "F.Cu") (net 4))
 (segment (start 7.112 -9.398) (end 10.16 -6.35) (width 0.5) (layer "F.Cu") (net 4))
 (segment (start 2.54 -7.874) (end 2.54 -9.398) (width 0.5) (layer "F.Cu") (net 4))
 (segment (start 10.16 -6.35) (end 10.16 -1.27) (width 0.5) (layer "F.Cu") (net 4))
 (segment (start 2.54 -9.398) (end 2.54 -12.192) (width 0.5) (layer "F.Cu") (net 4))
 (segment (start -2.54 -20.32) (end -2.54 -17.78) (width 2) (layer "F.Cu") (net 4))
 (segment (start -0.63 -11.097) (end -0.963 -11.43) (width 0.5) (layer "F.Cu") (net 10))
 (segment (start -0.63 -8.92) (end -0.63 -11.097) (width 0.5) (layer "F.Cu") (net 10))
 (segment (start 0.32 -11.163) (end 0.587 -11.43) (width 0.5) (layer "F.Cu") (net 8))
 (segment (start 0.32 -8.194) (end 0.32 -8.92) (width 0.5) (layer "F.Cu") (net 8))
 (segment (start -0.254 -7.62) (end 0.32 -8.194) (width 0.5) (layer "F.Cu") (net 8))
 (segment (start -4.191 -6.4365) (end -4.191 -6.858) (width 0.5) (layer "F.Cu") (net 8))
 (segment (start 0.32 -8.92) (end 0.32 -11.163) (width 0.5) (layer "F.Cu") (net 8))
 (segment (start -3.429 -7.62) (end -0.254 -7.62) (width 0.5) (layer "F.Cu") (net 8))
 (segment (start -4.2775 -6.35) (end -4.191 -6.4365) (width 0.5) (layer "F.Cu") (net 8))
 (segment (start -4.191 -6.858) (end -3.429 -7.62) (width 0.5) (layer "F.Cu") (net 8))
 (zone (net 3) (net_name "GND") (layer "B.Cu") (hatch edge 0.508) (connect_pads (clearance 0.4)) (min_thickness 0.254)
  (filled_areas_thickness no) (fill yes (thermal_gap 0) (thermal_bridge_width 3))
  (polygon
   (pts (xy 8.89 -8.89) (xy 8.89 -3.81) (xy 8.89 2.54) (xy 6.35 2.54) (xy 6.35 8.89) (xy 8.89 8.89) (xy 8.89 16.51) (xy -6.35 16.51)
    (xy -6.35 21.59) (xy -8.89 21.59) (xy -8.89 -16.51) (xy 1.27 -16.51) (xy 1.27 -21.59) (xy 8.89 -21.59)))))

